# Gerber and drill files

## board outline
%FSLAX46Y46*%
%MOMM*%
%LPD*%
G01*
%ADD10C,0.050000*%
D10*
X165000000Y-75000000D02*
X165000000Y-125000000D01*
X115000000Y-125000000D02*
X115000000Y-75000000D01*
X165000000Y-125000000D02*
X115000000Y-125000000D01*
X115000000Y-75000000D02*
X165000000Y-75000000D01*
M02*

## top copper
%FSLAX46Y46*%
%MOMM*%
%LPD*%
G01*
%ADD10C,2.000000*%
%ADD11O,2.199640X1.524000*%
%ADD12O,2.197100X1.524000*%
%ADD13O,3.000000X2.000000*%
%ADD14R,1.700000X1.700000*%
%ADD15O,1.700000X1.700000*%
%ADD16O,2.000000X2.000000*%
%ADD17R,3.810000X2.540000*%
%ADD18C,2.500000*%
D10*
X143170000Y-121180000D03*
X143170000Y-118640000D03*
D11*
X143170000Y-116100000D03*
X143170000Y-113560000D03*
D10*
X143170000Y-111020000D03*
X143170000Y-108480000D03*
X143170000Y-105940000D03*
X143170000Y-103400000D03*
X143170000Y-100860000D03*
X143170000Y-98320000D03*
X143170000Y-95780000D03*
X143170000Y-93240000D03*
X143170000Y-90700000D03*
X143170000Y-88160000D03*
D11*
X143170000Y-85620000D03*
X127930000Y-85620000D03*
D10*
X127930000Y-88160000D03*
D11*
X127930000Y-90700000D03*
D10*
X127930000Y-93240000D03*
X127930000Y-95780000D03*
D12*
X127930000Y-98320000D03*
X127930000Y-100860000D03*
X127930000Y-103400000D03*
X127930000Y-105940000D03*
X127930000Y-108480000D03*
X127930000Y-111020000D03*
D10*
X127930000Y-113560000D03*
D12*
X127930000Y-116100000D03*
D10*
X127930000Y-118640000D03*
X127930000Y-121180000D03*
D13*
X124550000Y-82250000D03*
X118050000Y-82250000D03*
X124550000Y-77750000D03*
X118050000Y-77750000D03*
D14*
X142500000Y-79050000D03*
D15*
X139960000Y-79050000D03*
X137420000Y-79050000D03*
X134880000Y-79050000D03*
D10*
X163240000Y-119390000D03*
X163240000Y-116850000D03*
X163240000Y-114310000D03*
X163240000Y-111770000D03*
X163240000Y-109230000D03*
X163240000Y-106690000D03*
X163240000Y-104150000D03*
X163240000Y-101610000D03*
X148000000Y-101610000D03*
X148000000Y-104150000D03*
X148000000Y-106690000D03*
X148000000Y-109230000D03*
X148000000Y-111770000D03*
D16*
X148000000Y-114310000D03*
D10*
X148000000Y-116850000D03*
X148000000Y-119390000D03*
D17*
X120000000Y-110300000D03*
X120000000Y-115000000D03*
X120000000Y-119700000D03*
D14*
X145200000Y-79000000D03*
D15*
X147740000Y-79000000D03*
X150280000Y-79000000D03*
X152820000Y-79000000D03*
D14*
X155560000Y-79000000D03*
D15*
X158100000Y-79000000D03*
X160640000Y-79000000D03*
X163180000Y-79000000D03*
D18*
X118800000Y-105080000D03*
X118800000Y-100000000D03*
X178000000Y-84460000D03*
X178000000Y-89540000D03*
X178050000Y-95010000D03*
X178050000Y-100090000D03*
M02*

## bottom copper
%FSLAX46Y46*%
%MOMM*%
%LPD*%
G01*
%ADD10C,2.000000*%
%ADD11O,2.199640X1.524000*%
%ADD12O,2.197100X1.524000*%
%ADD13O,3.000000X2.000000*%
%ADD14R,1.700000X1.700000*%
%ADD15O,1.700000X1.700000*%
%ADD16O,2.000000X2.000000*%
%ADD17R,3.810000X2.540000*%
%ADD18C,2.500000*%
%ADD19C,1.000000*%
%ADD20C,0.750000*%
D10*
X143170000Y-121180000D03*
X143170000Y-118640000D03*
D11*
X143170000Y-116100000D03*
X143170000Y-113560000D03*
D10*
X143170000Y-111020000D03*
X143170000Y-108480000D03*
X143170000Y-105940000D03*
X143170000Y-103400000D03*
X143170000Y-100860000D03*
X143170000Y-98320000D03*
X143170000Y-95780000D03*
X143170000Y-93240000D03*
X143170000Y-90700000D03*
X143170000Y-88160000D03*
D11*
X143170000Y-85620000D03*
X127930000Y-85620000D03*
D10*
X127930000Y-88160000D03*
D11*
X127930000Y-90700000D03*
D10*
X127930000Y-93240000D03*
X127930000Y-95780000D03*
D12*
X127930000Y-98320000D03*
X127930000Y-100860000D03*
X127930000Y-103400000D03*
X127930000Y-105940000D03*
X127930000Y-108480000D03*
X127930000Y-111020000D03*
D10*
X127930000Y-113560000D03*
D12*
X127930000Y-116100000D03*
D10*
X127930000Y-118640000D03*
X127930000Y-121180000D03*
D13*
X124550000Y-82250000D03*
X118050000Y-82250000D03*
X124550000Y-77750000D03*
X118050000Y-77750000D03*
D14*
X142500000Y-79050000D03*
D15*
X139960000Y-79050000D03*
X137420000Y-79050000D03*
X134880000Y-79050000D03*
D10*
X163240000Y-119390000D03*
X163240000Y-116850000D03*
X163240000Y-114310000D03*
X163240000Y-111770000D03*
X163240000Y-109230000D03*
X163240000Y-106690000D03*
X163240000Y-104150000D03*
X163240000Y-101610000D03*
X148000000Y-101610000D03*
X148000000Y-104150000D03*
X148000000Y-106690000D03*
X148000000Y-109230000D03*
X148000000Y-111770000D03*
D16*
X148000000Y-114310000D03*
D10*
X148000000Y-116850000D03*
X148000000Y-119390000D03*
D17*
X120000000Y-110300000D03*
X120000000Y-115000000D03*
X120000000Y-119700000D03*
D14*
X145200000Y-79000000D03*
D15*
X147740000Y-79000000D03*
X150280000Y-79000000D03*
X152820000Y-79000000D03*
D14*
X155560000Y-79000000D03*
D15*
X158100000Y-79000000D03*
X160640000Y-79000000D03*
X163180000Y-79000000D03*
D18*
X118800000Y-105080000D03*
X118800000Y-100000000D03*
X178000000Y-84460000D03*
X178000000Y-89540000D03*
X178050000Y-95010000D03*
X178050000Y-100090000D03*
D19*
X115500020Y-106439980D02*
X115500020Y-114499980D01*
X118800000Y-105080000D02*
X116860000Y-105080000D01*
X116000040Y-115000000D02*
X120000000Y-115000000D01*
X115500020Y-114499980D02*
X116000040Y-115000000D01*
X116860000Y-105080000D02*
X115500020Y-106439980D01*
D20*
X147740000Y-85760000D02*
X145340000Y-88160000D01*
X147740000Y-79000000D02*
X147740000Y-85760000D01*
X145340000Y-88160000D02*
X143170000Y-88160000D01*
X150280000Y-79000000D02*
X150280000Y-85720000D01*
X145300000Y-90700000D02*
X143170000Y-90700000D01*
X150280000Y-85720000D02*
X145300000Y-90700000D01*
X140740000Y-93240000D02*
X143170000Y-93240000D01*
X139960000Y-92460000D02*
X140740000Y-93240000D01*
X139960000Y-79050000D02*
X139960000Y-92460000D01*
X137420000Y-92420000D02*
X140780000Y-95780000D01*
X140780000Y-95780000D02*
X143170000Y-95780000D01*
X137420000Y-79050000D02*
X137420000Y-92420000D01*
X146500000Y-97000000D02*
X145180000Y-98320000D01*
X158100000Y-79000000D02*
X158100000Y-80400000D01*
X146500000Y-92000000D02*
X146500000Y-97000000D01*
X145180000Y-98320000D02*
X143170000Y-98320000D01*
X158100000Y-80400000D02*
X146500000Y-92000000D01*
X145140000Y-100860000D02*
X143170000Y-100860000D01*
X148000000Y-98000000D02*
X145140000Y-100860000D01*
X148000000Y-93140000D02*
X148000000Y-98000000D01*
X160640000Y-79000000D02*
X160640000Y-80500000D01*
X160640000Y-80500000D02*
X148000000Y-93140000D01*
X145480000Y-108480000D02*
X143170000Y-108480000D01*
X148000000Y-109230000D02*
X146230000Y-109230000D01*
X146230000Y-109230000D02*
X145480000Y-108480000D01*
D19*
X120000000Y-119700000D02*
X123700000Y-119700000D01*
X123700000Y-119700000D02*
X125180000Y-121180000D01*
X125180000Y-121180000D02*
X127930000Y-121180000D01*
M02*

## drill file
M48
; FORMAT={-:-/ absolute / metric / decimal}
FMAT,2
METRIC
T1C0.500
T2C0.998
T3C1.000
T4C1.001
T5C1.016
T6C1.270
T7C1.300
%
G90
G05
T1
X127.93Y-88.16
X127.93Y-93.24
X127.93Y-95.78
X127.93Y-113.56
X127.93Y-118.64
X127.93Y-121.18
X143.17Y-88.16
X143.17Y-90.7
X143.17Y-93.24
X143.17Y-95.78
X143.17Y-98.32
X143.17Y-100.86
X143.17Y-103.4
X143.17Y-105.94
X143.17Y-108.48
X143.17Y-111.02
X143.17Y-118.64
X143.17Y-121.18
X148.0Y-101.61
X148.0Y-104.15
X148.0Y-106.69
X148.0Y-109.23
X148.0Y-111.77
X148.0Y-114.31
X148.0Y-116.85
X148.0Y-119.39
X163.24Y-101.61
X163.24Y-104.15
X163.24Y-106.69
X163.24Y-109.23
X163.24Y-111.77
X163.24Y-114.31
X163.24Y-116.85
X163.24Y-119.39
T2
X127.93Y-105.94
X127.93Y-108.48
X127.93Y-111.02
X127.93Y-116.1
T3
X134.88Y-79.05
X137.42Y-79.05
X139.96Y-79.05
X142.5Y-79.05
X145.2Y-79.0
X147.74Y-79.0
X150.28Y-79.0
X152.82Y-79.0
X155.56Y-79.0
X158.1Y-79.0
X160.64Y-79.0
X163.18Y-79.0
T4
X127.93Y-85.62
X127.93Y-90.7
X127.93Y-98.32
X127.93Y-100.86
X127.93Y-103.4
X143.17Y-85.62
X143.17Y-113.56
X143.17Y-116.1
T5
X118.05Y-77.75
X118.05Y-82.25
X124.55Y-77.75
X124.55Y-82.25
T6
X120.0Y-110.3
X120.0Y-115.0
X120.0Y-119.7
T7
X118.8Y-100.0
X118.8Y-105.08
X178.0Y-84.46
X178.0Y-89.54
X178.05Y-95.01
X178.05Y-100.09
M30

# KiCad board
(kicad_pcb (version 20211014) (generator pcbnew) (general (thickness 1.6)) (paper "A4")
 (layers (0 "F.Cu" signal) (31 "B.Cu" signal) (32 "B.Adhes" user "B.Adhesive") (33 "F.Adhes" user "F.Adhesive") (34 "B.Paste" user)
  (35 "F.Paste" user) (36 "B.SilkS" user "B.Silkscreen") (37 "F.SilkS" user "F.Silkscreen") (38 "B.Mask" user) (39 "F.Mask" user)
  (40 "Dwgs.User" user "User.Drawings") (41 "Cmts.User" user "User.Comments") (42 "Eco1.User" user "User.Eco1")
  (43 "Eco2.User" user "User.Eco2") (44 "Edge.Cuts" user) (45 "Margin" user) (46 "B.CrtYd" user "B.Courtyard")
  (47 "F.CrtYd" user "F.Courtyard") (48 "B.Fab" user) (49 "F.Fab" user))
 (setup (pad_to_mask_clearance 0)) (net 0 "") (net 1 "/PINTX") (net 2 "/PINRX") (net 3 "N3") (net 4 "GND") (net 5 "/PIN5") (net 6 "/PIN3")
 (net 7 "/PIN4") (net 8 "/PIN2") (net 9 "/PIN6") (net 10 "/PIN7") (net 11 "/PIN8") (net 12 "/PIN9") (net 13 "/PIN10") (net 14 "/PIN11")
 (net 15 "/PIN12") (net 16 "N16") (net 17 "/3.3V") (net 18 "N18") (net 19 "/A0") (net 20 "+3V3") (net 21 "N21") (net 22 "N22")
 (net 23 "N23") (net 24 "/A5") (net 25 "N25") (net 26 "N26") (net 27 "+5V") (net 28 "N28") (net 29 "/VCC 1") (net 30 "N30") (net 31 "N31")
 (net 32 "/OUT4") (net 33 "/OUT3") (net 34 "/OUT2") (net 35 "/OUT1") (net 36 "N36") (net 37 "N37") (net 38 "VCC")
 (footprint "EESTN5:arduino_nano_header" (layer "F.Cu") (at 135.55 103.4 90)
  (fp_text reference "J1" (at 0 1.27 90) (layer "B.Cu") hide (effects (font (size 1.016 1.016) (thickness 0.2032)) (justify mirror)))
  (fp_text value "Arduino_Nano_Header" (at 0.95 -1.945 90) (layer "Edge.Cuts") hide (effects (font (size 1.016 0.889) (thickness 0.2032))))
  (pad "1" thru_hole circle locked (at -17.78 7.62 90) (size 2 2) (drill 0.5) (layers *.Cu *.Mask "F.SilkS") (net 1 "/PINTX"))
  (pad "2" thru_hole circle locked (at -15.24 7.62 90) (size 2 2) (drill 0.5) (layers *.Cu *.Mask "F.SilkS") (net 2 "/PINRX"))
  (pad "3" thru_hole oval locked (at -12.7 7.62 90) (size 1.524 2.19964) (drill 1.00076) (layers *.Cu *.Mask "F.SilkS") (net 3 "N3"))
  (pad "4" thru_hole oval locked (at -10.16 7.62 90) (size 1.524 2.19964) (drill 1.00076) (layers *.Cu *.Mask "F.SilkS") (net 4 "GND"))
  (pad "5" thru_hole circle locked (at -7.62 7.62 90) (size 2 2) (drill 0.5) (layers *.Cu *.Mask "F.SilkS") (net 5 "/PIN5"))
  (pad "6" thru_hole circle locked (at -5.08 7.62 90) (size 2 2) (drill 0.5) (layers *.Cu *.Mask "F.SilkS") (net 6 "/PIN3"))
  (pad "7" thru_hole circle locked (at -2.54 7.62 90) (size 2 2) (drill 0.5) (layers *.Cu *.Mask "F.SilkS") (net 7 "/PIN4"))
  (pad "8" thru_hole circle locked (at 0 7.62 90) (size 2 2) (drill 0.5) (layers *.Cu *.Mask "F.SilkS") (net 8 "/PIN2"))
  (pad "9" thru_hole circle locked (at 2.54 7.62 90) (size 2 2) (drill 0.5) (layers *.Cu *.Mask "F.SilkS") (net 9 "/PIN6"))
  (pad "10" thru_hole circle locked (at 5.08 7.62 90) (size 2 2) (drill 0.5) (layers *.Cu *.Mask "F.SilkS") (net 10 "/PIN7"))
  (pad "11" thru_hole circle locked (at 7.62 7.62 90) (size 2 2) (drill 0.5) (layers *.Cu *.Mask "F.SilkS") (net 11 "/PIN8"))
  (pad "12" thru_hole circle locked (at 10.16 7.62 90) (size 2 2) (drill 0.5) (layers *.Cu *.Mask "F.SilkS") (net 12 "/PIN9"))
  (pad "13" thru_hole circle locked (at 12.7 7.62 90) (size 2 2) (drill 0.5) (layers *.Cu *.Mask "F.SilkS") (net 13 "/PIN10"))
  (pad "14" thru_hole circle locked (at 15.24 7.62 90) (size 2 2) (drill 0.5) (layers *.Cu *.Mask "F.SilkS") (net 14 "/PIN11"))
  (pad "15" thru_hole oval locked (at 17.78 7.62 90) (size 1.524 2.19964) (drill 1.00076) (layers *.Cu *.Mask "F.SilkS") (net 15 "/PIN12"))
  (pad "16" thru_hole oval locked (at 17.78 -7.62 90) (size 1.524 2.19964) (drill 1.00076) (layers *.Cu *.Mask "F.SilkS") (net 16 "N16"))
  (pad "17" thru_hole circle locked (at 15.24 -7.62 90) (size 2 2) (drill 0.5) (layers *.Cu *.Mask "F.SilkS") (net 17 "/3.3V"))
  (pad "18" thru_hole oval locked (at 12.7 -7.62 90) (size 1.524 2.19964) (drill 1.00076) (layers *.Cu *.Mask "F.SilkS") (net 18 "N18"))
  (pad "19" thru_hole circle locked (at 10.16 -7.62 90) (size 2 2) (drill 0.5) (layers *.Cu *.Mask "F.SilkS") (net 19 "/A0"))
  (pad "20" thru_hole circle locked (at 7.62 -7.62 90) (size 2 2) (drill 0.5) (layers *.Cu *.Mask "F.SilkS") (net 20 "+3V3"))
  (pad "21" thru_hole oval locked (at 5.08 -7.62 90) (size 1.524 2.1971) (drill 1.00076) (layers *.Cu *.Mask "F.SilkS") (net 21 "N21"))
  (pad "22" thru_hole oval locked (at 2.54 -7.62 90) (size 1.524 2.1971) (drill 1.00076) (layers *.Cu *.Mask "F.SilkS") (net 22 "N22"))
  (pad "23" thru_hole oval locked (at 0 -7.62 90) (size 1.524 2.1971) (drill 1.00076) (layers *.Cu *.Mask "F.SilkS") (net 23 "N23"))
  (pad "24" thru_hole oval locked (at -2.54 -7.62 90) (size 1.524 2.1971) (drill 0.99822) (layers *.Cu *.Mask "F.SilkS") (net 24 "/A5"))
  (pad "25" thru_hole oval locked (at -5.08 -7.62 90) (size 1.524 2.1971) (drill 0.99822) (layers *.Cu *.Mask "F.SilkS") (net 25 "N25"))
  (pad "26" thru_hole oval locked (at -7.62 -7.62 90) (size 1.524 2.1971) (drill 0.99822) (layers *.Cu *.Mask "F.SilkS") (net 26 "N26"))
  (pad "27" thru_hole circle locked (at -10.16 -7.62 90) (size 2 2) (drill 0.5) (layers *.Cu *.Mask "F.SilkS") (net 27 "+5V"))
  (pad "28" thru_hole oval locked (at -12.7 -7.62 90) (size 1.524 2.1971) (drill 0.99822) (layers *.Cu *.Mask "F.SilkS") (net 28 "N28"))
  (pad "29" thru_hole circle locked (at -15.24 -7.62 90) (size 2 2) (drill 0.5) (layers *.Cu *.Mask "F.SilkS") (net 4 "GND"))
  (pad "30" thru_hole circle locked (at -17.78 -7.62 90) (size 2 2) (drill 0.5) (layers *.Cu *.Mask "F.SilkS") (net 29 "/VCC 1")))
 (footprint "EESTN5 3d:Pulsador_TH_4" (layer "F.Cu") (at 121.3 80 -90)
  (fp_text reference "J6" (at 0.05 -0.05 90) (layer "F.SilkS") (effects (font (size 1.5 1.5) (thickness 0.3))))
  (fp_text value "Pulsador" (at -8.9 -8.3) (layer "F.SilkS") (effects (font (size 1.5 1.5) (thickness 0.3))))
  (pad "1" thru_hole oval locked (at 2.25 -3.25 270) (size 2 3) (drill 1.016) (layers *.Cu *.Mask "F.SilkS") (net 24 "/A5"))
  (pad "2" thru_hole oval locked (at 2.25 3.25 270) (size 2 3) (drill 1.016) (layers *.Cu *.Mask "F.SilkS") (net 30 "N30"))
  (pad "3" thru_hole oval locked (at -2.25 -3.25 270) (size 2 3) (drill 1.016) (layers *.Cu *.Mask "F.SilkS") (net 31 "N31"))
  (pad "4" thru_hole oval locked (at -2.25 3.25 270) (size 2 3) (drill 1.016) (layers *.Cu *.Mask "F.SilkS") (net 4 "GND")))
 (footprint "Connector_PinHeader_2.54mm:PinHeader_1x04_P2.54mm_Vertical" (layer "F.Cu") (at 142.5 79.05 -90)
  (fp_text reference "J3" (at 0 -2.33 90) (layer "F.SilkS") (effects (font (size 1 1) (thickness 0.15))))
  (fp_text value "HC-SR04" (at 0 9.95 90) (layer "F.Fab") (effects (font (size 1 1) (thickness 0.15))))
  (pad "1" thru_hole rect (at 0 0 270) (size 1.7 1.7) (drill 1) (layers *.Cu *.Mask) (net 27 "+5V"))
  (pad "2" thru_hole oval (at 0 2.54 270) (size 1.7 1.7) (drill 1) (layers *.Cu *.Mask) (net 12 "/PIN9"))
  (pad "3" thru_hole oval (at 0 5.08 270) (size 1.7 1.7) (drill 1) (layers *.Cu *.Mask) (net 11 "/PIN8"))
  (pad "4" thru_hole oval (at 0 7.62 270) (size 1.7 1.7) (drill 1) (layers *.Cu *.Mask) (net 4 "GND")))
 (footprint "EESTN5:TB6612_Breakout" (layer "F.Cu") (at 155.62 110.5 90)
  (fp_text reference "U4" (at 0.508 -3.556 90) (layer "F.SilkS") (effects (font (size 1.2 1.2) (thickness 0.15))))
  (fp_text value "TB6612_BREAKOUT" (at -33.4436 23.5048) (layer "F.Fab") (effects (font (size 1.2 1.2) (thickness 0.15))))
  (pad "1" thru_hole circle locked (at -8.89 7.62 90) (size 2 2) (drill 0.5) (layers *.Cu *.Mask "F.SilkS") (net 29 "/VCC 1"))
  (pad "2" thru_hole circle locked (at -6.35 7.62 90) (size 2 2) (drill 0.5) (layers *.Cu *.Mask "F.SilkS") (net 27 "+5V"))
  (pad "3" thru_hole circle locked (at -3.81 7.62 90) (size 2 2) (drill 0.5) (layers *.Cu *.Mask "F.SilkS") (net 4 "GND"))
  (pad "4" thru_hole circle locked (at -1.27 7.62 90) (size 2 2) (drill 0.5) (layers *.Cu *.Mask "F.SilkS") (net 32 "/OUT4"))
  (pad "5" thru_hole circle locked (at 1.27 7.62 90) (size 2 2) (drill 0.5) (layers *.Cu *.Mask "F.SilkS") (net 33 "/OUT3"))
  (pad "6" thru_hole circle locked (at 3.81 7.62 90) (size 2 2) (drill 0.5) (layers *.Cu *.Mask "F.SilkS") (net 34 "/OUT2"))
  (pad "7" thru_hole circle locked (at 6.35 7.62 90) (size 2 2) (drill 0.5) (layers *.Cu *.Mask "F.SilkS") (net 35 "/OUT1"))
  (pad "8" thru_hole circle locked (at 8.89 7.62 90) (size 2 2) (drill 0.5) (layers *.Cu *.Mask "F.SilkS") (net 4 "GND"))
  (pad "9" thru_hole circle locked (at 8.89 -7.62 90) (size 2 2) (drill 0.5) (layers *.Cu *.Mask "F.SilkS") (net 4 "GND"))
  (pad "10" thru_hole circle locked (at 6.35 -7.62 90) (size 2 2) (drill 0.5) (layers *.Cu *.Mask "F.SilkS") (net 27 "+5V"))
  (pad "11" thru_hole circle locked (at 3.81 -7.62 90) (size 2 2) (drill 0.5) (layers *.Cu *.Mask "F.SilkS") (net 8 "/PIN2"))
  (pad "12" thru_hole circle locked (at 1.27 -7.62 90) (size 2 2) (drill 0.5) (layers *.Cu *.Mask "F.SilkS") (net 6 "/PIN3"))
  (pad "13" thru_hole circle locked (at -1.27 -7.62 90) (size 2 2) (drill 0.5) (layers *.Cu *.Mask "F.SilkS") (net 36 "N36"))
  (pad "14" thru_hole oval locked (at -3.81 -7.62 90) (size 2 2) (drill oval 0.5) (layers *.Cu *.Mask "F.SilkS") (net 7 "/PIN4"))
  (pad "15" thru_hole circle locked (at -6.35 -7.62 90) (size 2 2) (drill 0.5) (layers *.Cu *.Mask "F.SilkS") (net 5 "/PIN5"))
  (pad "16" thru_hole circle locked (at -8.89 -7.62 90) (size 2 2) (drill 0.5) (layers *.Cu *.Mask "F.SilkS") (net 27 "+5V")))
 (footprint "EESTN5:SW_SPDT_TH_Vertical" (layer "F.Cu") (at 120 115)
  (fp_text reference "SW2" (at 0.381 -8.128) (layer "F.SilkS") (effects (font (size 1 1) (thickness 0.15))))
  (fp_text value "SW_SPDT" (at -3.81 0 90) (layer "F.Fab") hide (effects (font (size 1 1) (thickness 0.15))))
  (pad "1" thru_hole rect locked (at 0 -4.7) (size 3.81 2.54) (drill 1.27) (layers *.Cu *.Mask) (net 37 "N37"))
  (pad "2" thru_hole rect locked (at 0 0) (size 3.81 2.54) (drill 1.27) (layers *.Cu *.Mask) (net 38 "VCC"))
  (pad "3" thru_hole rect locked (at 0 4.7) (size 3.81 2.54) (drill 1.27) (layers *.Cu *.Mask) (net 29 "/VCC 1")))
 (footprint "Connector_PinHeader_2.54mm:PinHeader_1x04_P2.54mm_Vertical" (layer "F.Cu") (at 145.2 79 90)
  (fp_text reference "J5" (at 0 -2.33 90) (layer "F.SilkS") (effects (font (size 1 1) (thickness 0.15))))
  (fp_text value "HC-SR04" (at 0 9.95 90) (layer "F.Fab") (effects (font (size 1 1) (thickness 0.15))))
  (pad "1" thru_hole rect (at 0 0 90) (size 1.7 1.7) (drill 1) (layers *.Cu *.Mask) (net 27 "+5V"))
  (pad "2" thru_hole oval (at 0 2.54 90) (size 1.7 1.7) (drill 1) (layers *.Cu *.Mask) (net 14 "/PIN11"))
  (pad "3" thru_hole oval (at 0 5.08 90) (size 1.7 1.7) (drill 1) (layers *.Cu *.Mask) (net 13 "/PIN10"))
  (pad "4" thru_hole oval (at 0 7.62 90) (size 1.7 1.7) (drill 1) (layers *.Cu *.Mask) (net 4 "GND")))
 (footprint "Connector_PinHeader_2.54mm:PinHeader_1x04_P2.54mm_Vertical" (layer "F.Cu") (at 155.56 79 90)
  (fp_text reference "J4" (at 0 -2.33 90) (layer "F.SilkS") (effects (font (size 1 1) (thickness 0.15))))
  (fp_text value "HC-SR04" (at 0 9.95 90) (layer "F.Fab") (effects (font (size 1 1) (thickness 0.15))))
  (pad "1" thru_hole rect (at 0 0 90) (size 1.7 1.7) (drill 1) (layers *.Cu *.Mask) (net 27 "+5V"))
  (pad "2" thru_hole oval (at 0 2.54 90) (size 1.7 1.7) (drill 1) (layers *.Cu *.Mask) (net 10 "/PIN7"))
  (pad "3" thru_hole oval (at 0 5.08 90) (size 1.7 1.7) (drill 1) (layers *.Cu *.Mask) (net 9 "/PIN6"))
  (pad "4" thru_hole oval (at 0 7.62 90) (size 1.7 1.7) (drill 1) (layers *.Cu *.Mask) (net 4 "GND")))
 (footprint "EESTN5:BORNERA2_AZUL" (layer "B.Cu") (at 118.8 102.54 90)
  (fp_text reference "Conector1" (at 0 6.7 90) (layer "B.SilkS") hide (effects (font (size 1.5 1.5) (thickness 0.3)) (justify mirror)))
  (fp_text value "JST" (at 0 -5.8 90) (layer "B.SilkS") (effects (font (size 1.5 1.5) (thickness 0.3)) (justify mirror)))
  (pad "1" thru_hole circle locked (at -2.54 0 90) (size 2.5 2.5) (drill 1.3) (layers *.Cu *.Mask "B.SilkS") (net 38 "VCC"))
  (pad "2" thru_hole circle locked (at 2.54 0 90) (size 2.5 2.5) (drill 1.3) (layers *.Cu *.Mask "B.SilkS") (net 4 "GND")))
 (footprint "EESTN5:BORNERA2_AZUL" (layer "B.Cu") (at 178 87 -90)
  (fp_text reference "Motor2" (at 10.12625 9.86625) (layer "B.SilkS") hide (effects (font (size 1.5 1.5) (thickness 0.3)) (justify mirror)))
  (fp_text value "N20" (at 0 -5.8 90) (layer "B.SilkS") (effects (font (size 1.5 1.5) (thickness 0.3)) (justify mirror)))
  (pad "1" thru_hole circle locked (at -2.54 0 270) (size 2.5 2.5) (drill 1.3) (layers *.Cu *.Mask "B.SilkS") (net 32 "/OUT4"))
  (pad "2" thru_hole circle locked (at 2.54 0 270) (size 2.5 2.5) (drill 1.3) (layers *.Cu *.Mask "B.SilkS") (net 33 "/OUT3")))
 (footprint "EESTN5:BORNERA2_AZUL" (layer "B.Cu") (at 178.05 97.55 -90)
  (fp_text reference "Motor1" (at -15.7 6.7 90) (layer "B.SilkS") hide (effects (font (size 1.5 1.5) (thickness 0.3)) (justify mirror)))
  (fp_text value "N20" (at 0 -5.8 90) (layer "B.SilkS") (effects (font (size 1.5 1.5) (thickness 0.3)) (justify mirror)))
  (pad "1" thru_hole circle locked (at -2.54 0 270) (size 2.5 2.5) (drill 1.3) (layers *.Cu *.Mask "B.SilkS") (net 34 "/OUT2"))
  (pad "2" thru_hole circle locked (at 2.54 0 270) (size 2.5 2.5) (drill 1.3) (layers *.Cu *.Mask "B.SilkS") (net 35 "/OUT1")))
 (gr_line (start 165 75) (end 165 125) (layer "Edge.Cuts") (width 0.05))
 (gr_line (start 115 125) (end 115 75) (layer "Edge.Cuts") (width 0.05))
 (gr_line (start 165 125) (end 115 125) (layer "Edge.Cuts") (width 0.05))
 (gr_line (start 115 75) (end 165 75) (layer "Edge.Cuts") (width 0.05))
 (segment (start 115.50002 106.43998) (end 115.50002 114.49998) (width 1) (layer "B.Cu") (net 38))
 (segment (start 118.8 105.08) (end 116.86 105.08) (width 1) (layer "B.Cu") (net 38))
 (segment (start 116.00004 115) (end 120 115) (width 1) (layer "B.Cu") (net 38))
 (segment (start 115.50002 114.49998) (end 116.00004 115) (width 1) (layer "B.Cu") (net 38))
 (segment (start 116.86 105.08) (end 115.50002 106.43998) (width 1) (layer "B.Cu") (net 38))
 (segment (start 147.74 85.76) (end 145.34 88.16) (width 0.75) (layer "B.Cu") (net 14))
 (segment (start 147.74 79) (end 147.74 85.76) (width 0.75) (layer "B.Cu") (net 14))
 (segment (start 145.34 88.16) (end 143.17 88.16) (width 0.75) (layer "B.Cu") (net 14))
 (segment (start 150.28 79) (end 150.28 85.72) (width 0.75) (layer "B.Cu") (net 13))
 (segment (start 145.3 90.7) (end 143.17 90.7) (width 0.75) (layer "B.Cu") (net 13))
 (segment (start 150.28 85.72) (end 145.3 90.7) (width 0.75) (layer "B.Cu") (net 13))
 (segment (start 140.74 93.24) (end 143.17 93.24) (width 0.75) (layer "B.Cu") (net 12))
 (segment (start 139.96 92.46) (end 140.74 93.24) (width 0.75) (layer "B.Cu") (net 12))
 (segment (start 139.96 79.05) (end 139.96 92.46) (width 0.75) (layer "B.Cu") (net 12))
 (segment (start 137.42 92.42) (end 140.78 95.78) (width 0.75) (layer "B.Cu") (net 11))
 (segment (start 140.78 95.78) (end 143.17 95.78) (width 0.75) (layer "B.Cu") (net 11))
 (segment (start 137.42 79.05) (end 137.42 92.42) (width 0.75) (layer "B.Cu") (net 11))
 (segment (start 146.5 97) (end 145.18 98.32) (width 0.75) (layer "B.Cu") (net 10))
 (segment (start 158.1 79) (end 158.1 80.4) (width 0.75) (layer "B.Cu") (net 10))
 (segment (start 146.5 92) (end 146.5 97) (width 0.75) (layer "B.Cu") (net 10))
 (segment (start 145.18 98.32) (end 143.17 98.32) (width 0.75) (layer "B.Cu") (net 10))
 (segment (start 158.1 80.4) (end 146.5 92) (width 0.75) (layer "B.Cu") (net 10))
 (segment (start 145.14 100.86) (end 143.17 100.86) (width 0.75) (layer "B.Cu") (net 9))
 (segment (start 148 98) (end 145.14 100.86) (width 0.75) (layer "B.Cu") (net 9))
 (segment (start 148 93.14) (end 148 98) (width 0.75) (layer "B.Cu") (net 9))
 (segment (start 160.64 79) (end 160.64 80.5) (width 0.75) (layer "B.Cu") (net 9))
 (segment (start 160.64 80.5) (end 148 93.14) (width 0.75) (layer "B.Cu") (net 9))
 (segment (start 145.48 108.48) (end 143.17 108.48) (width 0.75) (layer "B.Cu") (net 6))
 (segment (start 148 109.23) (end 146.23 109.23) (width 0.75) (layer "B.Cu") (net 6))
 (segment (start 146.23 109.23) (end 145.48 108.48) (width 0.75) (layer "B.Cu") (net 6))
 (segment (start 120 119.7) (end 123.7 119.7) (width 1) (layer "B.Cu") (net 29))
 (segment (start 123.7 119.7) (end 125.18 121.18) (width 1) (layer "B.Cu") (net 29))
 (segment (start 125.18 121.18) (end 127.93 121.18) (width 1) (layer "B.Cu") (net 29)))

